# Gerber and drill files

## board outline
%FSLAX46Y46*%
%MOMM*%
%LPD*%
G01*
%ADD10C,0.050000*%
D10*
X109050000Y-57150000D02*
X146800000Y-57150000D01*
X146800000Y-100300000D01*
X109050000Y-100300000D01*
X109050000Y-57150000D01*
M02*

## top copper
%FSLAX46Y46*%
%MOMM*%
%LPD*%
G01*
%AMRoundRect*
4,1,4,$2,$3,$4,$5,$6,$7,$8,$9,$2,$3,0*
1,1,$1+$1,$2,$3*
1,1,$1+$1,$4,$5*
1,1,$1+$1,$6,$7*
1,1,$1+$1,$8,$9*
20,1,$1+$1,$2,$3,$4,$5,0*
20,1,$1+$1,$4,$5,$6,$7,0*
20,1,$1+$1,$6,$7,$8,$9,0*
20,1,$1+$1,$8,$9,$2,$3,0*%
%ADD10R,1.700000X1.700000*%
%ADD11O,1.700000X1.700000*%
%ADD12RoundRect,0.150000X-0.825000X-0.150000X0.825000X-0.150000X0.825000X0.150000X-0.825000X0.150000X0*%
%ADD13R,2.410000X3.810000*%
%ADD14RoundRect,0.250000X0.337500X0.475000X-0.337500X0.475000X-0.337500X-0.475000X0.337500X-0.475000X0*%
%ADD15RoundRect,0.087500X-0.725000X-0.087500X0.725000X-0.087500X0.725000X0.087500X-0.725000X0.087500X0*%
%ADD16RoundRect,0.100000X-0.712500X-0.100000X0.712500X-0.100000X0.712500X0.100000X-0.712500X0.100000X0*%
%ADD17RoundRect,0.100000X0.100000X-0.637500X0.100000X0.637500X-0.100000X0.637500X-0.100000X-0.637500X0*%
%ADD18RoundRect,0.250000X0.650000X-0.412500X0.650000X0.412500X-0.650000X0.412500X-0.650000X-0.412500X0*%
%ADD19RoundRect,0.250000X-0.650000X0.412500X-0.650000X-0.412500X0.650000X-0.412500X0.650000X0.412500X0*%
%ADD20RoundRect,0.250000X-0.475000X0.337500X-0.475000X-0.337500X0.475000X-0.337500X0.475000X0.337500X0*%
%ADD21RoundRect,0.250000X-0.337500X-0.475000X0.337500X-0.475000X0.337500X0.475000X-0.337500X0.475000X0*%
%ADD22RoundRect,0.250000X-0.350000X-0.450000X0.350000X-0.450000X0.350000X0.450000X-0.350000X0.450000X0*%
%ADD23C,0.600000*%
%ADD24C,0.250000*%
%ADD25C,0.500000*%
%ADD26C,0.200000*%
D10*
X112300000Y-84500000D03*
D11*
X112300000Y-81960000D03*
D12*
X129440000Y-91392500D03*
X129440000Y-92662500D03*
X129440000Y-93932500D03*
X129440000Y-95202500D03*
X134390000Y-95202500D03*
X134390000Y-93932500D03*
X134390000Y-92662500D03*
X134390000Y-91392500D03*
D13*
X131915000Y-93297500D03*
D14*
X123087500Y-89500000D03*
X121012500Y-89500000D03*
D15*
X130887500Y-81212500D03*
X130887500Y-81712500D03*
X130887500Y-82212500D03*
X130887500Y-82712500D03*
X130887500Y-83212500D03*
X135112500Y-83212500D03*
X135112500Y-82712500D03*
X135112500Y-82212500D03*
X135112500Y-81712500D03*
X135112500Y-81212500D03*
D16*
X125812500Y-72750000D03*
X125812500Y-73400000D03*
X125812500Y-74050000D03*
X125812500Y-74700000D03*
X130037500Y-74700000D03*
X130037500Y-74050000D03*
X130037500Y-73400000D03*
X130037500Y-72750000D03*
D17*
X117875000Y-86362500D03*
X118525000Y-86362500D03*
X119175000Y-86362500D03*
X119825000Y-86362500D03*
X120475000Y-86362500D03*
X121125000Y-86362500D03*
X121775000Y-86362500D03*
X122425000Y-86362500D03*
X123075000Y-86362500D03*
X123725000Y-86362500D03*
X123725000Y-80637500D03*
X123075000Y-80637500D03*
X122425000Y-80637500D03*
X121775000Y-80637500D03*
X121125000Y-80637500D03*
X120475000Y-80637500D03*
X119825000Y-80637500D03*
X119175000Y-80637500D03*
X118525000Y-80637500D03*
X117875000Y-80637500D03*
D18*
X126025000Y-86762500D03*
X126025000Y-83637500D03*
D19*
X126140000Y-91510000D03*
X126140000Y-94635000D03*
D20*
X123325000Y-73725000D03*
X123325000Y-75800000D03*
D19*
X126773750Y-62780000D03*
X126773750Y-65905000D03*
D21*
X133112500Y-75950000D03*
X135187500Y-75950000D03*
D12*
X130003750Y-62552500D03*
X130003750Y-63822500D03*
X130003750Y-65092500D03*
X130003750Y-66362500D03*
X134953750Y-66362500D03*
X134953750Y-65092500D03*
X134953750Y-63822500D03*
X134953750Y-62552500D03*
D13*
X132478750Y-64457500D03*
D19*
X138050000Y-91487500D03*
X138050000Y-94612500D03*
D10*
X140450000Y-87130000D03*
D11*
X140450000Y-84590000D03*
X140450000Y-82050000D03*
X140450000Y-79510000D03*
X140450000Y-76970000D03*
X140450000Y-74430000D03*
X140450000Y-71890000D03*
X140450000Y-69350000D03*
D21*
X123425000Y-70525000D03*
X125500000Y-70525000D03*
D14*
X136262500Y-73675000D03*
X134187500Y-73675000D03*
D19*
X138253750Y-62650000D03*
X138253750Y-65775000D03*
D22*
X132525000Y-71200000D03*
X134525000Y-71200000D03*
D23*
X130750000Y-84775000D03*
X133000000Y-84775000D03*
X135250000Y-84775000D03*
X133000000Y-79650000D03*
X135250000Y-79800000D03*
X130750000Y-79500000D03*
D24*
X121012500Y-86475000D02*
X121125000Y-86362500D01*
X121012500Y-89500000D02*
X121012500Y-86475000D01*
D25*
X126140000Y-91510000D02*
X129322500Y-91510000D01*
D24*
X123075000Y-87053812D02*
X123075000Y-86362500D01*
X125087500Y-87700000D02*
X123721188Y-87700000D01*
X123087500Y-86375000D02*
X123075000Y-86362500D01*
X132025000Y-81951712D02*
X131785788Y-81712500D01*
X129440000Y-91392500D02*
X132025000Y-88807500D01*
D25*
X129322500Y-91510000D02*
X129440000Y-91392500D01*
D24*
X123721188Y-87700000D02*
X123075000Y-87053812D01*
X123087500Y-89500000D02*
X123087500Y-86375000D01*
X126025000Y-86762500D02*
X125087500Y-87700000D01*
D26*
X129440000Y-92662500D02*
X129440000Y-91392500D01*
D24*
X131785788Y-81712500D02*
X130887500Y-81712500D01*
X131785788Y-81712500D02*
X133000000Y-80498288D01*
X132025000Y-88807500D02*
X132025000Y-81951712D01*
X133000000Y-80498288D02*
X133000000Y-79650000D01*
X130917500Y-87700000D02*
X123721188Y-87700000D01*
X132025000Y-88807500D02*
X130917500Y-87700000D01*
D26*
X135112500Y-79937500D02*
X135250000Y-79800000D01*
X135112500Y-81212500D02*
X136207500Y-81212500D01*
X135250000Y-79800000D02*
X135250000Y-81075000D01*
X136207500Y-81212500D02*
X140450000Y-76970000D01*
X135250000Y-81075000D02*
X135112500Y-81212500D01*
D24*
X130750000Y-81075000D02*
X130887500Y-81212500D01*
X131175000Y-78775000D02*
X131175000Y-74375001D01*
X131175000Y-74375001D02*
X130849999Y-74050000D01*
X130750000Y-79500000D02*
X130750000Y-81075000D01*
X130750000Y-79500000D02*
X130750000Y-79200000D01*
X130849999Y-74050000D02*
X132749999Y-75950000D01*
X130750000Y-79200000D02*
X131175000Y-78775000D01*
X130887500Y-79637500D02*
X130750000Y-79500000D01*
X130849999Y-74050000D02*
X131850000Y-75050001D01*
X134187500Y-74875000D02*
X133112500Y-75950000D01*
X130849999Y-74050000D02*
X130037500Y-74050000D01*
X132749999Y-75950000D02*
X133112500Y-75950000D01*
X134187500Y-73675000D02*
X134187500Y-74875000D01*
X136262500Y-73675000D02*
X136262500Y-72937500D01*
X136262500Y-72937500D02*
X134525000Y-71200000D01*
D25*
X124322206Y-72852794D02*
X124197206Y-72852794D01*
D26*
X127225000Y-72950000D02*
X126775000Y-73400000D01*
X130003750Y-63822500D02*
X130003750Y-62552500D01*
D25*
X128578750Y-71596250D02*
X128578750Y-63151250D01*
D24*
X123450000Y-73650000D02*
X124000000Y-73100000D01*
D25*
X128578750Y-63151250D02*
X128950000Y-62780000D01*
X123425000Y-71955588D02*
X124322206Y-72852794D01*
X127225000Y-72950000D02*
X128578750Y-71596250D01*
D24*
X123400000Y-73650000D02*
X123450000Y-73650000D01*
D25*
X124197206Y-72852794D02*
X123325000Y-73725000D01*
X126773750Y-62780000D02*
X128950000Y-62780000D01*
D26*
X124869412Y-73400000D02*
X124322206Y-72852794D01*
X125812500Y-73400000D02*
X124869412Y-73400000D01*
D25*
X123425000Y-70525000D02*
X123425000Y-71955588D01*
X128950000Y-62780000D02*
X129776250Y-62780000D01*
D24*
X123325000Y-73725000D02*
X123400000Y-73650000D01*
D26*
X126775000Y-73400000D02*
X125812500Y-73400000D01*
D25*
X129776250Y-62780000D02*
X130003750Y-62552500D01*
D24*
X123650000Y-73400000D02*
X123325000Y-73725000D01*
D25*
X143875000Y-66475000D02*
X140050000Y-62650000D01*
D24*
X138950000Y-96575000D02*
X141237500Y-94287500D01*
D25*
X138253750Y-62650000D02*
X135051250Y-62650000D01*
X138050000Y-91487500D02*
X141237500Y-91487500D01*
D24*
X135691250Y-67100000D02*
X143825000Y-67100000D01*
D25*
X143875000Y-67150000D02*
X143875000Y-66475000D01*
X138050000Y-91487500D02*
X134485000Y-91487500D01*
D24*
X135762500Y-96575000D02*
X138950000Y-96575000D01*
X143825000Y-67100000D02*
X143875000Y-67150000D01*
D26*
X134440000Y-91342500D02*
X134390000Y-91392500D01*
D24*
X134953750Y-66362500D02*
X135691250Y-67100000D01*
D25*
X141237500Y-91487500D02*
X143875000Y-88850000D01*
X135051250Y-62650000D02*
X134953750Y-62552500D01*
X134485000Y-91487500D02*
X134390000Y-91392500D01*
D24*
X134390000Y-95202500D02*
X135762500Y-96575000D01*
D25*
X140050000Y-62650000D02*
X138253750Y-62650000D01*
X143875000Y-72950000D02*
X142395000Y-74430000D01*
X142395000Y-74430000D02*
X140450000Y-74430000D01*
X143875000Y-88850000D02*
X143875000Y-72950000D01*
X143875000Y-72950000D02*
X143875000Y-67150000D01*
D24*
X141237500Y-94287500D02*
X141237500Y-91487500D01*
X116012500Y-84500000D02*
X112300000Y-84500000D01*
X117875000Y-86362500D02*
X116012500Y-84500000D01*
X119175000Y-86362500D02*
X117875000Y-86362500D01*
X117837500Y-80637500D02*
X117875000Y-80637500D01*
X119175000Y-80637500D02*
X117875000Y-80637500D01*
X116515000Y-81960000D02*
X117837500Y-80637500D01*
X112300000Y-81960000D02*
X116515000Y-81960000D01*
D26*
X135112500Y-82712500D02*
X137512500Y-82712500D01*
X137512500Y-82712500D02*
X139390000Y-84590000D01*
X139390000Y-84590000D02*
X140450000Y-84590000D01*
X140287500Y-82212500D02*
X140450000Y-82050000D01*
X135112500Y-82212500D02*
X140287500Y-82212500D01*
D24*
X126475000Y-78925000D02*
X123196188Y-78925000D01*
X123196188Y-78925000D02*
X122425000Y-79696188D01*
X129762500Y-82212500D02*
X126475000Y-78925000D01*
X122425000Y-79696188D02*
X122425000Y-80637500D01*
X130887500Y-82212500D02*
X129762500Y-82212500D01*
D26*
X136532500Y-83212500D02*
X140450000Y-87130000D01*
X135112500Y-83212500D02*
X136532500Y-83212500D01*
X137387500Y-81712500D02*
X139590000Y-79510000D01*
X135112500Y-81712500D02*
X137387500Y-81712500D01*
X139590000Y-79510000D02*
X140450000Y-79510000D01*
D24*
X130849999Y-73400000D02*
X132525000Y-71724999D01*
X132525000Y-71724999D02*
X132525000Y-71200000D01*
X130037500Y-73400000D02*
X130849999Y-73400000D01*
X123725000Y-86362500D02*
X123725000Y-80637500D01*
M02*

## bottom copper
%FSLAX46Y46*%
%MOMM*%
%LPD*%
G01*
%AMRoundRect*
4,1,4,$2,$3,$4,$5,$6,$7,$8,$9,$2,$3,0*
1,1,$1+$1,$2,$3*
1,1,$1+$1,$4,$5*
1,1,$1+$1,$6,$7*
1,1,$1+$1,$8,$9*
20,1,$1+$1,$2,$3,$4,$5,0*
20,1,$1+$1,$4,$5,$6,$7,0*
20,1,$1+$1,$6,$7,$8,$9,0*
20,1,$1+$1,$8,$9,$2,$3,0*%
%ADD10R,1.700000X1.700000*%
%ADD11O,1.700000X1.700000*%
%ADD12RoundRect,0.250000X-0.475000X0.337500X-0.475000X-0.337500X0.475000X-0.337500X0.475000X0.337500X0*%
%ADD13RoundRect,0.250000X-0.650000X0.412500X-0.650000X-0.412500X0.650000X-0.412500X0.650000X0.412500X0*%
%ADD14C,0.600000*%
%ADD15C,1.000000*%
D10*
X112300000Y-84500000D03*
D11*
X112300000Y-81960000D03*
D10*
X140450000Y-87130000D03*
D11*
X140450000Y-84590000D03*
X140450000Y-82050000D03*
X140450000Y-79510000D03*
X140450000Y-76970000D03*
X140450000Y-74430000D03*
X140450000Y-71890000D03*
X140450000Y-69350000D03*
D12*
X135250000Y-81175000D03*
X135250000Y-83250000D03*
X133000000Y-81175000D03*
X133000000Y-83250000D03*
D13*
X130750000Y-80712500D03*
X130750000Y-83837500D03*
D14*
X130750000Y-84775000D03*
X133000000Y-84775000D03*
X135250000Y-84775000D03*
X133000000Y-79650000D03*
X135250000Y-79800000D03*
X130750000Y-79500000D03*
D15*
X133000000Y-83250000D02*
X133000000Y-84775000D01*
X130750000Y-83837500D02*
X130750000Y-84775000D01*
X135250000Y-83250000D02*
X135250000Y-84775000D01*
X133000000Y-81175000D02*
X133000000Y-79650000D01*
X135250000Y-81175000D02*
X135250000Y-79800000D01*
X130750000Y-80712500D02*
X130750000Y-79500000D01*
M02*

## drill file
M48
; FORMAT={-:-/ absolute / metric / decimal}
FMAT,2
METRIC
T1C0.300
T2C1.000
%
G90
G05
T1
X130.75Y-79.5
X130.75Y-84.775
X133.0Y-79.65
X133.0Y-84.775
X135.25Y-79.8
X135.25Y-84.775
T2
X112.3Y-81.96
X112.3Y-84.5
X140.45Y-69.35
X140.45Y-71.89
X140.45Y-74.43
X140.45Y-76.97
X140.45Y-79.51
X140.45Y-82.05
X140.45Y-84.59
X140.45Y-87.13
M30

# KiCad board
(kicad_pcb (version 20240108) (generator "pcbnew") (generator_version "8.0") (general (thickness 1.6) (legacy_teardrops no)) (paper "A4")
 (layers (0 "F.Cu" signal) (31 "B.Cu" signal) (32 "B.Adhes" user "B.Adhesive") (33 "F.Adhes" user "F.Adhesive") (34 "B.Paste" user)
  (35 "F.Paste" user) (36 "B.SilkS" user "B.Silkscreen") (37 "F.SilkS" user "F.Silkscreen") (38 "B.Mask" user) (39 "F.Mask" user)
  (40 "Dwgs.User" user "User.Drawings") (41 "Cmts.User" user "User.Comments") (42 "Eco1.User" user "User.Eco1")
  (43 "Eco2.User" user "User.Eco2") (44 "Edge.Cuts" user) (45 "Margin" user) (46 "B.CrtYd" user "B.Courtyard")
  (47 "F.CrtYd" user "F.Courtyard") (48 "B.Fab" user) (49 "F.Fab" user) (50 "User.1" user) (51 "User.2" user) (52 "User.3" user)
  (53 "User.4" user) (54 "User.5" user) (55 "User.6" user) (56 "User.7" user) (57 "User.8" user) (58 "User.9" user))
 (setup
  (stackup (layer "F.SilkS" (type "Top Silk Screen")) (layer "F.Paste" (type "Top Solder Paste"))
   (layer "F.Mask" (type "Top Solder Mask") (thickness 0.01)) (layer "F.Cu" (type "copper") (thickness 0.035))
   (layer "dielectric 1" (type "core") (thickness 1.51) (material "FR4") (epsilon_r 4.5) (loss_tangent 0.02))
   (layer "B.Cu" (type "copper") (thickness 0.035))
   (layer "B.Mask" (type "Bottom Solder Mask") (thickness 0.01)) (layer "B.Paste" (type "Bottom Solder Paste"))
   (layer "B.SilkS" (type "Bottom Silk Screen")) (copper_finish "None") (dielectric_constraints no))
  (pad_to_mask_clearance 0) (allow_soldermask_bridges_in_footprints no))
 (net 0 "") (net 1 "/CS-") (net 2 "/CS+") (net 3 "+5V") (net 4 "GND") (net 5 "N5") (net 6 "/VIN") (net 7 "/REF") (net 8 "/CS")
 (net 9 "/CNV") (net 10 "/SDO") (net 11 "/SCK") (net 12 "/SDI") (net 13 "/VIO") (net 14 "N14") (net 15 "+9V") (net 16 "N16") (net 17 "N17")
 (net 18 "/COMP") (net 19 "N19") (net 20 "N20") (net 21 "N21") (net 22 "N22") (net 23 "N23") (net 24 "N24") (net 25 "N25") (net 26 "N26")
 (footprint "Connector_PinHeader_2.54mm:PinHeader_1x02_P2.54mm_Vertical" (layer "F.Cu") (at 112.3 84.5 180)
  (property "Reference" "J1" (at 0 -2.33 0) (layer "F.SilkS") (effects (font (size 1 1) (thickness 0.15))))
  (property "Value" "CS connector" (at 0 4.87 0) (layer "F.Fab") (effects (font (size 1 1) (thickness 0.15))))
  (pad "1" thru_hole rect (at 0 0 180) (size 1.7 1.7) (drill 1) (layers "*.Cu" "*.Mask") (remove_unused_layers no) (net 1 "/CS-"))
  (pad "2" thru_hole oval (at 0 2.54 180) (size 1.7 1.7) (drill 1) (layers "*.Cu" "*.Mask") (remove_unused_layers no) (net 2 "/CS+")))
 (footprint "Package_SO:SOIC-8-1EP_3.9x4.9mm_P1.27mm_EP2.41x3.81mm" (layer "F.Cu") (at 131.915 93.2975)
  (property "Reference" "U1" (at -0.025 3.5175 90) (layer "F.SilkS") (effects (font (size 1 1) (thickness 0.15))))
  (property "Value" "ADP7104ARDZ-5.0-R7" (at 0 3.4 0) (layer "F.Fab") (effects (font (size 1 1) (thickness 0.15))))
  (pad "" smd roundrect (at -0.6 -0.95) (size 0.97 1.54) (layers "F.Paste") (roundrect_rratio 0.25))
  (pad "" smd roundrect (at -0.6 0.95) (size 0.97 1.54) (layers "F.Paste") (roundrect_rratio 0.25))
  (pad "" smd roundrect (at 0.6 -0.95) (size 0.97 1.54) (layers "F.Paste") (roundrect_rratio 0.25))
  (pad "" smd roundrect (at 0.6 0.95) (size 0.97 1.54) (layers "F.Paste") (roundrect_rratio 0.25))
  (pad "1" smd roundrect (at -2.475 -1.905) (size 1.95 0.6) (layers "F.Cu" "F.Paste" "F.Mask") (roundrect_rratio 0.25) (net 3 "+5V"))
  (pad "2" smd roundrect (at -2.475 -0.635) (size 1.95 0.6) (layers "F.Cu" "F.Paste" "F.Mask") (roundrect_rratio 0.25) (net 3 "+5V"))
  (pad "3" smd roundrect (at -2.475 0.635) (size 1.95 0.6) (layers "F.Cu" "F.Paste" "F.Mask") (roundrect_rratio 0.25) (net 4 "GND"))
  (pad "4" smd roundrect (at -2.475 1.905) (size 1.95 0.6) (layers "F.Cu" "F.Paste" "F.Mask") (roundrect_rratio 0.25) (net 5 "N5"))
  (pad "5" smd roundrect (at 2.475 1.905) (size 1.95 0.6) (layers "F.Cu" "F.Paste" "F.Mask") (roundrect_rratio 0.25) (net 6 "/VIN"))
  (pad "6" smd roundrect (at 2.475 0.635) (size 1.95 0.6) (layers "F.Cu" "F.Paste" "F.Mask") (roundrect_rratio 0.25) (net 4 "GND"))
  (pad "7" smd roundrect (at 2.475 -0.635) (size 1.95 0.6) (layers "F.Cu" "F.Paste" "F.Mask") (roundrect_rratio 0.25) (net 4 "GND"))
  (pad "8" smd roundrect (at 2.475 -1.905) (size 1.95 0.6) (layers "F.Cu" "F.Paste" "F.Mask") (roundrect_rratio 0.25) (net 6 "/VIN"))
  (pad "9" smd rect (at 0 0) (size 2.41 3.81) (layers "F.Cu" "F.Mask") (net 4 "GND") (zone_connect 2)))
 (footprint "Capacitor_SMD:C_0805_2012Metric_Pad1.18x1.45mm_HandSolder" (layer "F.Cu") (at 122.05 89.5 180)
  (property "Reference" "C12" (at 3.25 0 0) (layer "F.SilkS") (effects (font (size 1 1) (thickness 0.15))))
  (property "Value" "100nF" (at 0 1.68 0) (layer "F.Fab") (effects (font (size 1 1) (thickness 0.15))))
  (pad "1" smd roundrect (at -1.0375 0 180) (size 1.175 1.45) (layers "F.Cu" "F.Paste" "F.Mask") (roundrect_rratio 0.212766) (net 3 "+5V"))
  (pad "2" smd roundrect (at 1.0375 0 180) (size 1.175 1.45) (layers "F.Cu" "F.Paste" "F.Mask") (roundrect_rratio 0.212766) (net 4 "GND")))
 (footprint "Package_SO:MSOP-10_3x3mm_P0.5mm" (layer "F.Cu") (at 133 82.2125)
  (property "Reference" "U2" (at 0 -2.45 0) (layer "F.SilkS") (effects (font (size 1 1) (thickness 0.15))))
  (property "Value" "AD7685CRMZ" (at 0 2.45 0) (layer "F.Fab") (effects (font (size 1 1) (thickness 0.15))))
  (pad "1" smd roundrect (at -2.1125 -1) (size 1.625 0.35) (layers "F.Cu" "F.Paste" "F.Mask") (roundrect_rratio 0.25) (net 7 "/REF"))
  (pad "2" smd roundrect (at -2.1125 -0.5) (size 1.625 0.35) (layers "F.Cu" "F.Paste" "F.Mask") (roundrect_rratio 0.25) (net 3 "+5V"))
  (pad "3" smd roundrect (at -2.1125 0) (size 1.625 0.35) (layers "F.Cu" "F.Paste" "F.Mask") (roundrect_rratio 0.25) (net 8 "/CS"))
  (pad "4" smd roundrect (at -2.1125 0.5) (size 1.625 0.35) (layers "F.Cu" "F.Paste" "F.Mask") (roundrect_rratio 0.25) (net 4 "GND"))
  (pad "5" smd roundrect (at -2.1125 1) (size 1.625 0.35) (layers "F.Cu" "F.Paste" "F.Mask") (roundrect_rratio 0.25) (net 4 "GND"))
  (pad "6" smd roundrect (at 2.1125 1) (size 1.625 0.35) (layers "F.Cu" "F.Paste" "F.Mask") (roundrect_rratio 0.25) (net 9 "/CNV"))
  (pad "7" smd roundrect (at 2.1125 0.5) (size 1.625 0.35) (layers "F.Cu" "F.Paste" "F.Mask") (roundrect_rratio 0.25) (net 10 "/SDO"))
  (pad "8" smd roundrect (at 2.1125 0) (size 1.625 0.35) (layers "F.Cu" "F.Paste" "F.Mask") (roundrect_rratio 0.25) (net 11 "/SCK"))
  (pad "9" smd roundrect (at 2.1125 -0.5) (size 1.625 0.35) (layers "F.Cu" "F.Paste" "F.Mask") (roundrect_rratio 0.25) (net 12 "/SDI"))
  (pad "10" smd roundrect (at 2.1125 -1) (size 1.625 0.35) (layers "F.Cu" "F.Paste" "F.Mask") (roundrect_rratio 0.25) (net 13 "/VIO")))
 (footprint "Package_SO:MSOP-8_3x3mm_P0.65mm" (layer "F.Cu") (at 127.925 73.725)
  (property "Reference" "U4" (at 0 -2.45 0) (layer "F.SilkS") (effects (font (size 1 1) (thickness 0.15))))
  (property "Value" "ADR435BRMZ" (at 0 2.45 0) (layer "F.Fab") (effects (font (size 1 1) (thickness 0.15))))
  (pad "1" smd roundrect (at -2.1125 -0.975) (size 1.625 0.4) (layers "F.Cu" "F.Paste" "F.Mask") (roundrect_rratio 0.25) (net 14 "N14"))
  (pad "2" smd roundrect (at -2.1125 -0.325) (size 1.625 0.4) (layers "F.Cu" "F.Paste" "F.Mask") (roundrect_rratio 0.25) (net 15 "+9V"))
  (pad "3" smd roundrect (at -2.1125 0.325) (size 1.625 0.4) (layers "F.Cu" "F.Paste" "F.Mask") (roundrect_rratio 0.25) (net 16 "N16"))
  (pad "4" smd roundrect (at -2.1125 0.975) (size 1.625 0.4) (layers "F.Cu" "F.Paste" "F.Mask") (roundrect_rratio 0.25) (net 4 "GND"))
  (pad "5" smd roundrect (at 2.1125 0.975) (size 1.625 0.4) (layers "F.Cu" "F.Paste" "F.Mask") (roundrect_rratio 0.25) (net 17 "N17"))
  (pad "6" smd roundrect (at 2.1125 0.325) (size 1.625 0.4) (layers "F.Cu" "F.Paste" "F.Mask") (roundrect_rratio 0.25) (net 7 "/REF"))
  (pad "7" smd roundrect (at 2.1125 -0.325) (size 1.625 0.4) (layers "F.Cu" "F.Paste" "F.Mask") (roundrect_rratio 0.25) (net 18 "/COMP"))
  (pad "8" smd roundrect (at 2.1125 -0.975) (size 1.625 0.4) (layers "F.Cu" "F.Paste" "F.Mask") (roundrect_rratio 0.25) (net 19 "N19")))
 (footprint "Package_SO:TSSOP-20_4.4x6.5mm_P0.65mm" (layer "F.Cu") (at 120.8 83.5 90)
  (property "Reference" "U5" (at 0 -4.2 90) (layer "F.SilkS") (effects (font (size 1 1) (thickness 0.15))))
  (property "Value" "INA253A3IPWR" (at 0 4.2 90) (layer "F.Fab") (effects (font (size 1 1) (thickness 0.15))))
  (pad "1" smd roundrect (at -2.8625 -2.925 90) (size 1.475 0.4) (layers "F.Cu" "F.Paste" "F.Mask") (roundrect_rratio 0.25) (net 1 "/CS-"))
  (pad "2" smd roundrect (at -2.8625 -2.275 90) (size 1.475 0.4) (layers "F.Cu" "F.Paste" "F.Mask") (roundrect_rratio 0.25) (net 1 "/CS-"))
  (pad "3" smd roundrect (at -2.8625 -1.625 90) (size 1.475 0.4) (layers "F.Cu" "F.Paste" "F.Mask") (roundrect_rratio 0.25) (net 1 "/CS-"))
  (pad "4" smd roundrect (at -2.8625 -0.975 90) (size 1.475 0.4) (layers "F.Cu" "F.Paste" "F.Mask") (roundrect_rratio 0.25) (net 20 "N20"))
  (pad "5" smd roundrect (at -2.8625 -0.325 90) (size 1.475 0.4) (layers "F.Cu" "F.Paste" "F.Mask") (roundrect_rratio 0.25) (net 20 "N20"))
  (pad "6" smd roundrect (at -2.8625 0.325 90) (size 1.475 0.4) (layers "F.Cu" "F.Paste" "F.Mask") (roundrect_rratio 0.25) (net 4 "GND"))
  (pad "7" smd roundrect (at -2.8625 0.975 90) (size 1.475 0.4) (layers "F.Cu" "F.Paste" "F.Mask") (roundrect_rratio 0.25) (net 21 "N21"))
  (pad "8" smd roundrect (at -2.8625 1.625 90) (size 1.475 0.4) (layers "F.Cu" "F.Paste" "F.Mask") (roundrect_rratio 0.25) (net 4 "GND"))
  (pad "9" smd roundrect (at -2.8625 2.275 90) (size 1.475 0.4) (layers "F.Cu" "F.Paste" "F.Mask") (roundrect_rratio 0.25) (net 3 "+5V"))
  (pad "10" smd roundrect (at -2.8625 2.925 90) (size 1.475 0.4) (layers "F.Cu" "F.Paste" "F.Mask") (roundrect_rratio 0.25) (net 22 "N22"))
  (pad "11" smd roundrect (at 2.8625 2.925 90) (size 1.475 0.4) (layers "F.Cu" "F.Paste" "F.Mask") (roundrect_rratio 0.25) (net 22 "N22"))
  (pad "12" smd roundrect (at 2.8625 2.275 90) (size 1.475 0.4) (layers "F.Cu" "F.Paste" "F.Mask") (roundrect_rratio 0.25) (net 4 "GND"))
  (pad "13" smd roundrect (at 2.8625 1.625 90) (size 1.475 0.4) (layers "F.Cu" "F.Paste" "F.Mask") (roundrect_rratio 0.25) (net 8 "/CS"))
  (pad "14" smd roundrect (at 2.8625 0.975 90) (size 1.475 0.4) (layers "F.Cu" "F.Paste" "F.Mask") (roundrect_rratio 0.25) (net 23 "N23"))
  (pad "15" smd roundrect (at 2.8625 0.325 90) (size 1.475 0.4) (layers "F.Cu" "F.Paste" "F.Mask") (roundrect_rratio 0.25) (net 4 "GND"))
  (pad "16" smd roundrect (at 2.8625 -0.325 90) (size 1.475 0.4) (layers "F.Cu" "F.Paste" "F.Mask") (roundrect_rratio 0.25) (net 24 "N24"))
  (pad "17" smd roundrect (at 2.8625 -0.975 90) (size 1.475 0.4) (layers "F.Cu" "F.Paste" "F.Mask") (roundrect_rratio 0.25) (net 24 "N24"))
  (pad "18" smd roundrect (at 2.8625 -1.625 90) (size 1.475 0.4) (layers "F.Cu" "F.Paste" "F.Mask") (roundrect_rratio 0.25) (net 2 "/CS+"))
  (pad "19" smd roundrect (at 2.8625 -2.275 90) (size 1.475 0.4) (layers "F.Cu" "F.Paste" "F.Mask") (roundrect_rratio 0.25) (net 2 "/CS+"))
  (pad "20" smd roundrect (at 2.8625 -2.925 90) (size 1.475 0.4) (layers "F.Cu" "F.Paste" "F.Mask") (roundrect_rratio 0.25) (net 2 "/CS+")))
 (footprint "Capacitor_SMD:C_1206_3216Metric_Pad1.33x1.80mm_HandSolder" (layer "F.Cu") (at 126.025 85.2 90)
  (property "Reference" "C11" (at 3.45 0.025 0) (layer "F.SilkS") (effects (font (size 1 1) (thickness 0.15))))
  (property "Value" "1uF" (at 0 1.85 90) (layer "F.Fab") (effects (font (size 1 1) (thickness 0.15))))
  (pad "1" smd roundrect (at -1.5625 0 90) (size 1.325 1.8) (layers "F.Cu" "F.Paste" "F.Mask") (roundrect_rratio 0.188679) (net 3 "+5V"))
  (pad "2" smd roundrect (at 1.5625 0 90) (size 1.325 1.8) (layers "F.Cu" "F.Paste" "F.Mask") (roundrect_rratio 0.188679) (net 4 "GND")))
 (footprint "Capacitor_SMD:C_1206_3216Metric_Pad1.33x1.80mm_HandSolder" (layer "F.Cu") (at 126.14 93.0725 -90)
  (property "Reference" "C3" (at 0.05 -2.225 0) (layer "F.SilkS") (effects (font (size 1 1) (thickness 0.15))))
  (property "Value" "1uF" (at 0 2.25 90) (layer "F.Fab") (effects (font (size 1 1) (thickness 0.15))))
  (pad "1" smd roundrect (at -1.5625 0 270) (size 1.325 1.8) (layers "F.Cu" "F.Paste" "F.Mask") (roundrect_rratio 0.188679) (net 3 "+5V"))
  (pad "2" smd roundrect (at 1.5625 0 270) (size 1.325 1.8) (layers "F.Cu" "F.Paste" "F.Mask") (roundrect_rratio 0.188679) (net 4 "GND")))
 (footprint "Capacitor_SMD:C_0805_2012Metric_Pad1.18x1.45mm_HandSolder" (layer "F.Cu") (at 123.325 74.7625 -90)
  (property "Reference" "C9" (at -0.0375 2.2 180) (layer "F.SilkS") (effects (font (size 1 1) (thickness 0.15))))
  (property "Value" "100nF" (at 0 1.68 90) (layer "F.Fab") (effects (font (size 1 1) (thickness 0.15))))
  (pad "1" smd roundrect (at -1.0375 0 270) (size 1.175 1.45) (layers "F.Cu" "F.Paste" "F.Mask") (roundrect_rratio 0.212766) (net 15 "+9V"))
  (pad "2" smd roundrect (at 1.0375 0 270) (size 1.175 1.45) (layers "F.Cu" "F.Paste" "F.Mask") (roundrect_rratio 0.212766) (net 4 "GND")))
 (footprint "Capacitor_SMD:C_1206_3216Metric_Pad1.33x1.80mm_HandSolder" (layer "F.Cu") (at 126.77375 64.3425 -90)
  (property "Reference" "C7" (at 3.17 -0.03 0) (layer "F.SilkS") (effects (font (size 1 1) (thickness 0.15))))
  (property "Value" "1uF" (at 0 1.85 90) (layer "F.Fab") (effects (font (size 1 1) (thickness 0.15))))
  (pad "1" smd roundrect (at -1.5625 0 270) (size 1.325 1.8) (layers "F.Cu" "F.Paste" "F.Mask") (roundrect_rratio 0.188679) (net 15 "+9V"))
  (pad "2" smd roundrect (at 1.5625 0 270) (size 1.325 1.8) (layers "F.Cu" "F.Paste" "F.Mask") (roundrect_rratio 0.188679) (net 4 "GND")))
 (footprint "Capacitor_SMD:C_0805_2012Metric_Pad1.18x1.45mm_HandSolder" (layer "F.Cu") (at 134.15 75.95)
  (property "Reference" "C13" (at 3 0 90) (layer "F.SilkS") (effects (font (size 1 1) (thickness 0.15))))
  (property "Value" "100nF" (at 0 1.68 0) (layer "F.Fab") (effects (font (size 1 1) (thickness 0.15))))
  (pad "1" smd roundrect (at -1.0375 0) (size 1.175 1.45) (layers "F.Cu" "F.Paste" "F.Mask") (roundrect_rratio 0.212766) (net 7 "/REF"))
  (pad "2" smd roundrect (at 1.0375 0) (size 1.175 1.45) (layers "F.Cu" "F.Paste" "F.Mask") (roundrect_rratio 0.212766) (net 4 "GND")))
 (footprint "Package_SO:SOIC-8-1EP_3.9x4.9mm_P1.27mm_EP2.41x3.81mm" (layer "F.Cu") (at 132.47875 64.4575)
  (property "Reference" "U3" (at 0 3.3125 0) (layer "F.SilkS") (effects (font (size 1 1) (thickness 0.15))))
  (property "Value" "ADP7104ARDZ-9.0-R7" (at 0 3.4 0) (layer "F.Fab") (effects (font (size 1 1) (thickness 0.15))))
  (pad "" smd roundrect (at -0.6 -0.95) (size 0.97 1.54) (layers "F.Paste") (roundrect_rratio 0.25))
  (pad "" smd roundrect (at -0.6 0.95) (size 0.97 1.54) (layers "F.Paste") (roundrect_rratio 0.25))
  (pad "" smd roundrect (at 0.6 -0.95) (size 0.97 1.54) (layers "F.Paste") (roundrect_rratio 0.25))
  (pad "" smd roundrect (at 0.6 0.95) (size 0.97 1.54) (layers "F.Paste") (roundrect_rratio 0.25))
  (pad "1" smd roundrect (at -2.475 -1.905) (size 1.95 0.6) (layers "F.Cu" "F.Paste" "F.Mask") (roundrect_rratio 0.25) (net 15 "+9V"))
  (pad "2" smd roundrect (at -2.475 -0.635) (size 1.95 0.6) (layers "F.Cu" "F.Paste" "F.Mask") (roundrect_rratio 0.25) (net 15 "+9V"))
  (pad "3" smd roundrect (at -2.475 0.635) (size 1.95 0.6) (layers "F.Cu" "F.Paste" "F.Mask") (roundrect_rratio 0.25) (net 4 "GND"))
  (pad "4" smd roundrect (at -2.475 1.905) (size 1.95 0.6) (layers "F.Cu" "F.Paste" "F.Mask") (roundrect_rratio 0.25) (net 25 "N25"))
  (pad "5" smd roundrect (at 2.475 1.905) (size 1.95 0.6) (layers "F.Cu" "F.Paste" "F.Mask") (roundrect_rratio 0.25) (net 6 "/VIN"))
  (pad "6" smd roundrect (at 2.475 0.635) (size 1.95 0.6) (layers "F.Cu" "F.Paste" "F.Mask") (roundrect_rratio 0.25) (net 4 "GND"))
  (pad "7" smd roundrect (at 2.475 -0.635) (size 1.95 0.6) (layers "F.Cu" "F.Paste" "F.Mask") (roundrect_rratio 0.25) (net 4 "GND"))
  (pad "8" smd roundrect (at 2.475 -1.905) (size 1.95 0.6) (layers "F.Cu" "F.Paste" "F.Mask") (roundrect_rratio 0.25) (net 6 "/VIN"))
  (pad "9" smd rect (at 0 0) (size 2.41 3.81) (layers "F.Cu" "F.Mask") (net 4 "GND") (zone_connect 2)))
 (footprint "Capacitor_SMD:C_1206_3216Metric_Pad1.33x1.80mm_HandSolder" (layer "F.Cu") (at 138.05 93.05 -90)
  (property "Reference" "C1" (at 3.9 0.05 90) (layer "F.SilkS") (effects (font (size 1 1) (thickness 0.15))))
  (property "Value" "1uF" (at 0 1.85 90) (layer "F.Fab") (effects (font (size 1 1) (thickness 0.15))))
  (pad "1" smd roundrect (at -1.5625 0 270) (size 1.325 1.8) (layers "F.Cu" "F.Paste" "F.Mask") (roundrect_rratio 0.188679) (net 6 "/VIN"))
  (pad "2" smd roundrect (at 1.5625 0 270) (size 1.325 1.8) (layers "F.Cu" "F.Paste" "F.Mask") (roundrect_rratio 0.188679) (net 4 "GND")))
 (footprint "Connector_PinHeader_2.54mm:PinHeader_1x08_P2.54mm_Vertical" (layer "F.Cu") (at 140.45 87.13 180)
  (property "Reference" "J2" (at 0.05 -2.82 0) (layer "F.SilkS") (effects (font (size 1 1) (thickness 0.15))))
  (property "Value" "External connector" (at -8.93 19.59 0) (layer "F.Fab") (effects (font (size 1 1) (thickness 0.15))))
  (pad "1" thru_hole rect (at 0 0 180) (size 1.7 1.7) (drill 1) (layers "*.Cu" "*.Mask") (remove_unused_layers no) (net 9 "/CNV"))
  (pad "2" thru_hole oval (at 0 2.54 180) (size 1.7 1.7) (drill 1) (layers "*.Cu" "*.Mask") (remove_unused_layers no) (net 10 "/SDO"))
  (pad "3" thru_hole oval (at 0 5.08 180) (size 1.7 1.7) (drill 1) (layers "*.Cu" "*.Mask") (remove_unused_layers no) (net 11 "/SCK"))
  (pad "4" thru_hole oval (at 0 7.62 180) (size 1.7 1.7) (drill 1) (layers "*.Cu" "*.Mask") (remove_unused_layers no) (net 12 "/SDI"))
  (pad "5" thru_hole oval (at 0 10.16 180) (size 1.7 1.7) (drill 1) (layers "*.Cu" "*.Mask") (remove_unused_layers no) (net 13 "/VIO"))
  (pad "6" thru_hole oval (at 0 12.7 180) (size 1.7 1.7) (drill 1) (layers "*.Cu" "*.Mask") (remove_unused_layers no) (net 6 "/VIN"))
  (pad "7" thru_hole oval (at 0 15.24 180) (size 1.7 1.7) (drill 1) (layers "*.Cu" "*.Mask") (remove_unused_layers no) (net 4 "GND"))
  (pad "8" thru_hole oval (at 0 17.78 180) (size 1.7 1.7) (drill 1) (layers "*.Cu" "*.Mask") (remove_unused_layers no) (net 8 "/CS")))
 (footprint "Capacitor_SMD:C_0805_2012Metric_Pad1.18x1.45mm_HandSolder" (layer "F.Cu") (at 124.4625 70.525)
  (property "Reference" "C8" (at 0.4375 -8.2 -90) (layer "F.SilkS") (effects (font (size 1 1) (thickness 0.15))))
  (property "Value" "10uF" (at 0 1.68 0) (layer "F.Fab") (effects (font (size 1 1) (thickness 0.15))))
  (pad "1" smd roundrect (at -1.0375 0) (size 1.175 1.45) (layers "F.Cu" "F.Paste" "F.Mask") (roundrect_rratio 0.212766) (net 15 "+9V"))
  (pad "2" smd roundrect (at 1.0375 0) (size 1.175 1.45) (layers "F.Cu" "F.Paste" "F.Mask") (roundrect_rratio 0.212766) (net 4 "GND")))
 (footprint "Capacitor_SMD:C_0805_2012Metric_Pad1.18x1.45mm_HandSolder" (layer "F.Cu") (at 135.225 73.675 180)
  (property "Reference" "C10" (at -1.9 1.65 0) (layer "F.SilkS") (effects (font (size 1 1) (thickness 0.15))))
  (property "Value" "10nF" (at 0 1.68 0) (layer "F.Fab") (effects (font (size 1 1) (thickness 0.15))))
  (pad "1" smd roundrect (at -1.0375 0 180) (size 1.175 1.45) (layers "F.Cu" "F.Paste" "F.Mask") (roundrect_rratio 0.212766) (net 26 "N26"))
  (pad "2" smd roundrect (at 1.0375 0 180) (size 1.175 1.45) (layers "F.Cu" "F.Paste" "F.Mask") (roundrect_rratio 0.212766) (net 7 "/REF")))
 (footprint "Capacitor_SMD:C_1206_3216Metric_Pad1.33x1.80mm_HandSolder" (layer "F.Cu") (at 138.25375 64.2125 -90)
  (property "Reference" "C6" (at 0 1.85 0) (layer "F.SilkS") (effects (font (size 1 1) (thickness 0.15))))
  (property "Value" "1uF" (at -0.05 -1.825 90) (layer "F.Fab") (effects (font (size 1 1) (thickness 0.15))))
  (pad "1" smd roundrect (at -1.5625 0 270) (size 1.325 1.8) (layers "F.Cu" "F.Paste" "F.Mask") (roundrect_rratio 0.188679) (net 6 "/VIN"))
  (pad "2" smd roundrect (at 1.5625 0 270) (size 1.325 1.8) (layers "F.Cu" "F.Paste" "F.Mask") (roundrect_rratio 0.188679) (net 4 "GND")))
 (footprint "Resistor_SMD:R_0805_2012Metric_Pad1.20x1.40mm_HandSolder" (layer "F.Cu") (at 133.525 71.2)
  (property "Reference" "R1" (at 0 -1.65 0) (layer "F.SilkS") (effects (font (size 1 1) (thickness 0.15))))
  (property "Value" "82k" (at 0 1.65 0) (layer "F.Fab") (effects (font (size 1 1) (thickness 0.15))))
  (pad "1" smd roundrect (at -1 0) (size 1.2 1.4) (layers "F.Cu" "F.Paste" "F.Mask") (roundrect_rratio 0.208333) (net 18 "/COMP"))
  (pad "2" smd roundrect (at 1 0) (size 1.2 1.4) (layers "F.Cu" "F.Paste" "F.Mask") (roundrect_rratio 0.208333) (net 26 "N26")))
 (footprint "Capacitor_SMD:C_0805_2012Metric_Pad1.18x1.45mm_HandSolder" (layer "B.Cu") (at 135.25 82.2125 -90)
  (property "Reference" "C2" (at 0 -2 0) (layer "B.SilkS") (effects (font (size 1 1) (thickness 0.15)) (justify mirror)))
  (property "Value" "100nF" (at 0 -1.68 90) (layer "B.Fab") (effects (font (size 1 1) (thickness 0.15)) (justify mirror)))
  (pad "1" smd roundrect (at -1.0375 0 270) (size 1.175 1.45) (layers "B.Cu" "B.Paste" "B.Mask") (roundrect_rratio 0.212766) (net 13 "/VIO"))
  (pad "2" smd roundrect (at 1.0375 0 270) (size 1.175 1.45) (layers "B.Cu" "B.Paste" "B.Mask") (roundrect_rratio 0.212766) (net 4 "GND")))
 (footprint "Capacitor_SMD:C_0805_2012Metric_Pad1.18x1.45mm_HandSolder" (layer "B.Cu") (at 133 82.2125 -90)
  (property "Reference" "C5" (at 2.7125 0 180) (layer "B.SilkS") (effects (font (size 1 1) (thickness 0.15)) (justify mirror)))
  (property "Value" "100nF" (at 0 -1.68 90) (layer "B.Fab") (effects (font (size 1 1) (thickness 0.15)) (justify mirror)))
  (pad "1" smd roundrect (at -1.0375 0 270) (size 1.175 1.45) (layers "B.Cu" "B.Paste" "B.Mask") (roundrect_rratio 0.212766) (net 3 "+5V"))
  (pad "2" smd roundrect (at 1.0375 0 270) (size 1.175 1.45) (layers "B.Cu" "B.Paste" "B.Mask") (roundrect_rratio 0.212766) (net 4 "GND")))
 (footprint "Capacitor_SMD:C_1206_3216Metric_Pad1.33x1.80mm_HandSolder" (layer "B.Cu") (at 130.75 82.275 -90)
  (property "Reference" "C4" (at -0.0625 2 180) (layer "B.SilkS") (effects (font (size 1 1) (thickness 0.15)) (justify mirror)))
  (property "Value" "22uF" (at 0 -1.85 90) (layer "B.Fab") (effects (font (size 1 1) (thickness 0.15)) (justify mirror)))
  (pad "1" smd roundrect (at -1.5625 0 270) (size 1.325 1.8) (layers "B.Cu" "B.Paste" "B.Mask") (roundrect_rratio 0.188679) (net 7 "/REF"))
  (pad "2" smd roundrect (at 1.5625 0 270) (size 1.325 1.8) (layers "B.Cu" "B.Paste" "B.Mask") (roundrect_rratio 0.188679) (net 4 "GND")))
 (gr_rect (start 109.05 57.15) (end 146.8 100.3) (stroke (width 0.05) (type default)) (fill none) (layer "Edge.Cuts"))
 (segment (start 121.0125 86.475) (end 121.125 86.3625) (width 0.25) (layer "F.Cu") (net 4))
 (segment (start 121.0125 89.5) (end 121.0125 86.475) (width 0.25) (layer "F.Cu") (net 4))
 (via (at 130.75 84.775) (size 0.6) (drill 0.3) (layers "F.Cu" "B.Cu") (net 4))
 (via (at 133 84.775) (size 0.6) (drill 0.3) (layers "F.Cu" "B.Cu") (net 4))
 (via (at 135.25 84.775) (size 0.6) (drill 0.3) (layers "F.Cu" "B.Cu") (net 4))
 (segment (start 133 83.25) (end 133 84.775) (width 1) (layer "B.Cu") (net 4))
 (segment (start 130.75 83.8375) (end 130.75 84.775) (width 1) (layer "B.Cu") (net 4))
 (segment (start 135.25 83.25) (end 135.25 84.775) (width 1) (layer "B.Cu") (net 4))
 (segment (start 126.14 91.51) (end 129.3225 91.51) (width 0.5) (layer "F.Cu") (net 3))
 (segment (start 123.075 87.053812) (end 123.075 86.3625) (width 0.25) (layer "F.Cu") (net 3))
 (segment (start 125.0875 87.7) (end 123.721188 87.7) (width 0.25) (layer "F.Cu") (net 3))
 (segment (start 123.0875 86.375) (end 123.075 86.3625) (width 0.25) (layer "F.Cu") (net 3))
 (segment (start 132.025 81.951712) (end 131.785788 81.7125) (width 0.25) (layer "F.Cu") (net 3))
 (segment (start 129.44 91.3925) (end 132.025 88.8075) (width 0.25) (layer "F.Cu") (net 3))
 (segment (start 129.3225 91.51) (end 129.44 91.3925) (width 0.5) (layer "F.Cu") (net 3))
 (segment (start 123.721188 87.7) (end 123.075 87.053812) (width 0.25) (layer "F.Cu") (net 3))
 (segment (start 123.0875 89.5) (end 123.0875 86.375) (width 0.25) (layer "F.Cu") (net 3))
 (segment (start 126.025 86.7625) (end 125.0875 87.7) (width 0.25) (layer "F.Cu") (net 3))
 (segment (start 129.44 92.6625) (end 129.44 91.3925) (width 0.2) (layer "F.Cu") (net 3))
 (segment (start 131.785788 81.7125) (end 130.8875 81.7125) (width 0.25) (layer "F.Cu") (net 3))
 (segment (start 131.785788 81.7125) (end 133 80.498288) (width 0.25) (layer "F.Cu") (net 3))
 (segment (start 132.025 88.8075) (end 132.025 81.951712) (width 0.25) (layer "F.Cu") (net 3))
 (segment (start 133 80.498288) (end 133 79.65) (width 0.25) (layer "F.Cu") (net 3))
 (segment (start 130.9175 87.7) (end 123.721188 87.7) (width 0.25) (layer "F.Cu") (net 3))
 (segment (start 132.025 88.8075) (end 130.9175 87.7) (width 0.25) (layer "F.Cu") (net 3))
 (via (at 133 79.65) (size 0.6) (drill 0.3) (layers "F.Cu" "B.Cu") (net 3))
 (segment (start 133 81.175) (end 133 79.65) (width 1) (layer "B.Cu") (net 3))
 (segment (start 135.1125 79.9375) (end 135.25 79.8) (width 0.2) (layer "F.Cu") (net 13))
 (segment (start 135.1125 81.2125) (end 136.2075 81.2125) (width 0.2) (layer "F.Cu") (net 13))
 (segment (start 135.25 79.8) (end 135.25 81.075) (width 0.2) (layer "F.Cu") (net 13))
 (segment (start 136.2075 81.2125) (end 140.45 76.97) (width 0.2) (layer "F.Cu") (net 13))
 (segment (start 135.25 81.075) (end 135.1125 81.2125) (width 0.2) (layer "F.Cu") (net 13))
 (via (at 135.25 79.8) (size 0.6) (drill 0.3) (layers "F.Cu" "B.Cu") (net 13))
 (segment (start 135.25 81.175) (end 135.25 79.8) (width 1) (layer "B.Cu") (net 13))
 (segment (start 130.75 81.075) (end 130.8875 81.2125) (width 0.25) (layer "F.Cu") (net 7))
 (segment (start 131.175 78.775) (end 131.175 74.375001) (width 0.25) (layer "F.Cu") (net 7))
 (segment (start 131.175 74.375001) (end 130.849999 74.05) (width 0.25) (layer "F.Cu") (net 7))
 (segment (start 130.75 79.5) (end 130.75 81.075) (width 0.25) (layer "F.Cu") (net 7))
 (segment (start 130.75 79.5) (end 130.75 79.2) (width 0.25) (layer "F.Cu") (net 7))
 (segment (start 130.849999 74.05) (end 132.749999 75.95) (width 0.25) (layer "F.Cu") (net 7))
 (segment (start 130.75 79.2) (end 131.175 78.775) (width 0.25) (layer "F.Cu") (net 7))
 (segment (start 130.8875 79.6375) (end 130.75 79.5) (width 0.25) (layer "F.Cu") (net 7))
 (segment (start 130.849999 74.05) (end 131.85 75.050001) (width 0.25) (layer "F.Cu") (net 7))
 (segment (start 134.1875 74.875) (end 133.1125 75.95) (width 0.25) (layer "F.Cu") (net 7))
 (segment (start 130.849999 74.05) (end 130.0375 74.05) (width 0.25) (layer "F.Cu") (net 7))
 (segment (start 132.749999 75.95) (end 133.1125 75.95) (width 0.25) (layer "F.Cu") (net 7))
 (segment (start 134.1875 73.675) (end 134.1875 74.875) (width 0.25) (layer "F.Cu") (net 7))
 (via (at 130.75 79.5) (size 0.6) (drill 0.3) (layers "F.Cu" "B.Cu") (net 7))
 (segment (start 130.75 80.7125) (end 130.75 79.5) (width 1) (layer "B.Cu") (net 7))
 (segment (start 136.2625 73.675) (end 136.2625 72.9375) (width 0.25) (layer "F.Cu") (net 26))
 (segment (start 136.2625 72.9375) (end 134.525 71.2) (width 0.25) (layer "F.Cu") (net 26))
 (segment (start 124.322206 72.852794) (end 124.197206 72.852794) (width 0.5) (layer "F.Cu") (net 15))
 (segment (start 127.225 72.95) (end 126.775 73.4) (width 0.2) (layer "F.Cu") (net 15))
 (segment (start 130.00375 63.8225) (end 130.00375 62.5525) (width 0.2) (layer "F.Cu") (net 15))
 (segment (start 128.57875 71.59625) (end 128.57875 63.15125) (width 0.5) (layer "F.Cu") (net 15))
 (segment (start 123.45 73.65) (end 124 73.1) (width 0.25) (layer "F.Cu") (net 15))
 (segment (start 128.57875 63.15125) (end 128.95 62.78) (width 0.5) (layer "F.Cu") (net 15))
 (segment (start 123.425 71.955588) (end 124.322206 72.852794) (width 0.5) (layer "F.Cu") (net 15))
 (segment (start 127.225 72.95) (end 128.57875 71.59625) (width 0.5) (layer "F.Cu") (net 15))
 (segment (start 123.4 73.65) (end 123.45 73.65) (width 0.25) (layer "F.Cu") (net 15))
 (segment (start 124.197206 72.852794) (end 123.325 73.725) (width 0.5) (layer "F.Cu") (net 15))
 (segment (start 126.77375 62.78) (end 128.95 62.78) (width 0.5) (layer "F.Cu") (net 15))
 (segment (start 124.869412 73.4) (end 124.322206 72.852794) (width 0.2) (layer "F.Cu") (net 15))
 (segment (start 125.8125 73.4) (end 124.869412 73.4) (width 0.2) (layer "F.Cu") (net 15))
 (segment (start 123.425 70.525) (end 123.425 71.955588) (width 0.5) (layer "F.Cu") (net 15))
 (segment (start 128.95 62.78) (end 129.77625 62.78) (width 0.5) (layer "F.Cu") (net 15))
 (segment (start 123.325 73.725) (end 123.4 73.65) (width 0.25) (layer "F.Cu") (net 15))
 (segment (start 126.775 73.4) (end 125.8125 73.4) (width 0.2) (layer "F.Cu") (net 15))
 (segment (start 129.77625 62.78) (end 130.00375 62.5525) (width 0.5) (layer "F.Cu") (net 15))
 (segment (start 123.65 73.4) (end 123.325 73.725) (width 0.25) (layer "F.Cu") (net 15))
 (segment (start 143.875 66.475) (end 140.05 62.65) (width 0.5) (layer "F.Cu") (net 6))
 (segment (start 138.95 96.575) (end 141.2375 94.2875) (width 0.25) (layer "F.Cu") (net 6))
 (segment (start 138.25375 62.65) (end 135.05125 62.65) (width 0.5) (layer "F.Cu") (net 6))
 (segment (start 138.05 91.4875) (end 141.2375 91.4875) (width 0.5) (layer "F.Cu") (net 6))
 (segment (start 135.69125 67.1) (end 143.825 67.1) (width 0.25) (layer "F.Cu") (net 6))
 (segment (start 143.875 67.15) (end 143.875 66.475) (width 0.5) (layer "F.Cu") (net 6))
 (segment (start 138.05 91.4875) (end 134.485 91.4875) (width 0.5) (layer "F.Cu") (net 6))
 (segment (start 135.7625 96.575) (end 138.95 96.575) (width 0.25) (layer "F.Cu") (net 6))
 (segment (start 143.825 67.1) (end 143.875 67.15) (width 0.25) (layer "F.Cu") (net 6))
 (segment (start 134.44 91.3425) (end 134.39 91.3925) (width 0.2) (layer "F.Cu") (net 6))
 (segment (start 134.95375 66.3625) (end 135.69125 67.1) (width 0.25) (layer "F.Cu") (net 6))
 (segment (start 141.2375 91.4875) (end 143.875 88.85) (width 0.5) (layer "F.Cu") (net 6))
 (segment (start 135.05125 62.65) (end 134.95375 62.5525) (width 0.5) (layer "F.Cu") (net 6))
 (segment (start 134.485 91.4875) (end 134.39 91.3925) (width 0.5) (layer "F.Cu") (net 6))
 (segment (start 134.39 95.2025) (end 135.7625 96.575) (width 0.25) (layer "F.Cu") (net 6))
 (segment (start 140.05 62.65) (end 138.25375 62.65) (width 0.5) (layer "F.Cu") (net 6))
 (segment (start 143.875 72.95) (end 142.395 74.43) (width 0.5) (layer "F.Cu") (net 6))
 (segment (start 142.395 74.43) (end 140.45 74.43) (width 0.5) (layer "F.Cu") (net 6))
 (segment (start 143.875 88.85) (end 143.875 72.95) (width 0.5) (layer "F.Cu") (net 6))
 (segment (start 143.875 72.95) (end 143.875 67.15) (width 0.5) (layer "F.Cu") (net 6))
 (segment (start 141.2375 94.2875) (end 141.2375 91.4875) (width 0.25) (layer "F.Cu") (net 6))
 (segment (start 116.0125 84.5) (end 112.3 84.5) (width 0.25) (layer "F.Cu") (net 1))
 (segment (start 117.875 86.3625) (end 116.0125 84.5) (width 0.25) (layer "F.Cu") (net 1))
 (segment (start 119.175 86.3625) (end 117.875 86.3625) (width 0.25) (layer "F.Cu") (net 1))
 (segment (start 117.8375 80.6375) (end 117.875 80.6375) (width 0.25) (layer "F.Cu") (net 2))
 (segment (start 119.175 80.6375) (end 117.875 80.6375) (width 0.25) (layer "F.Cu") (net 2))
 (segment (start 116.515 81.96) (end 117.8375 80.6375) (width 0.25) (layer "F.Cu") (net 2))
 (segment (start 112.3 81.96) (end 116.515 81.96) (width 0.25) (layer "F.Cu") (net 2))
 (segment (start 135.1125 82.7125) (end 137.5125 82.7125) (width 0.2) (layer "F.Cu") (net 10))
 (segment (start 137.5125 82.7125) (end 139.39 84.59) (width 0.2) (layer "F.Cu") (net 10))
 (segment (start 139.39 84.59) (end 140.45 84.59) (width 0.2) (layer "F.Cu") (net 10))
 (segment (start 140.2875 82.2125) (end 140.45 82.05) (width 0.2) (layer "F.Cu") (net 11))
 (segment (start 135.1125 82.2125) (end 140.2875 82.2125) (width 0.2) (layer "F.Cu") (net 11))
 (segment (start 126.475 78.925) (end 123.196188 78.925) (width 0.25) (layer "F.Cu") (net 8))
 (segment (start 123.196188 78.925) (end 122.425 79.696188) (width 0.25) (layer "F.Cu") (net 8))
 (segment (start 129.7625 82.2125) (end 126.475 78.925) (width 0.25) (layer "F.Cu") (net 8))
 (segment (start 122.425 79.696188) (end 122.425 80.6375) (width 0.25) (layer "F.Cu") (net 8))
 (segment (start 130.8875 82.2125) (end 129.7625 82.2125) (width 0.25) (layer "F.Cu") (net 8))
 (segment (start 136.5325 83.2125) (end 140.45 87.13) (width 0.2) (layer "F.Cu") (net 9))
 (segment (start 135.1125 83.2125) (end 136.5325 83.2125) (width 0.2) (layer "F.Cu") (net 9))
 (segment (start 137.3875 81.7125) (end 139.59 79.51) (width 0.2) (layer "F.Cu") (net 12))
 (segment (start 135.1125 81.7125) (end 137.3875 81.7125) (width 0.2) (layer "F.Cu") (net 12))
 (segment (start 139.59 79.51) (end 140.45 79.51) (width 0.2) (layer "F.Cu") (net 12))
 (segment (start 130.849999 73.4) (end 132.525 71.724999) (width 0.25) (layer "F.Cu") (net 18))
 (segment (start 132.525 71.724999) (end 132.525 71.2) (width 0.25) (layer "F.Cu") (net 18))
 (segment (start 130.0375 73.4) (end 130.849999 73.4) (width 0.25) (layer "F.Cu") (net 18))
 (segment (start 123.725 86.3625) (end 123.725 80.6375) (width 0.25) (layer "F.Cu") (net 22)))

